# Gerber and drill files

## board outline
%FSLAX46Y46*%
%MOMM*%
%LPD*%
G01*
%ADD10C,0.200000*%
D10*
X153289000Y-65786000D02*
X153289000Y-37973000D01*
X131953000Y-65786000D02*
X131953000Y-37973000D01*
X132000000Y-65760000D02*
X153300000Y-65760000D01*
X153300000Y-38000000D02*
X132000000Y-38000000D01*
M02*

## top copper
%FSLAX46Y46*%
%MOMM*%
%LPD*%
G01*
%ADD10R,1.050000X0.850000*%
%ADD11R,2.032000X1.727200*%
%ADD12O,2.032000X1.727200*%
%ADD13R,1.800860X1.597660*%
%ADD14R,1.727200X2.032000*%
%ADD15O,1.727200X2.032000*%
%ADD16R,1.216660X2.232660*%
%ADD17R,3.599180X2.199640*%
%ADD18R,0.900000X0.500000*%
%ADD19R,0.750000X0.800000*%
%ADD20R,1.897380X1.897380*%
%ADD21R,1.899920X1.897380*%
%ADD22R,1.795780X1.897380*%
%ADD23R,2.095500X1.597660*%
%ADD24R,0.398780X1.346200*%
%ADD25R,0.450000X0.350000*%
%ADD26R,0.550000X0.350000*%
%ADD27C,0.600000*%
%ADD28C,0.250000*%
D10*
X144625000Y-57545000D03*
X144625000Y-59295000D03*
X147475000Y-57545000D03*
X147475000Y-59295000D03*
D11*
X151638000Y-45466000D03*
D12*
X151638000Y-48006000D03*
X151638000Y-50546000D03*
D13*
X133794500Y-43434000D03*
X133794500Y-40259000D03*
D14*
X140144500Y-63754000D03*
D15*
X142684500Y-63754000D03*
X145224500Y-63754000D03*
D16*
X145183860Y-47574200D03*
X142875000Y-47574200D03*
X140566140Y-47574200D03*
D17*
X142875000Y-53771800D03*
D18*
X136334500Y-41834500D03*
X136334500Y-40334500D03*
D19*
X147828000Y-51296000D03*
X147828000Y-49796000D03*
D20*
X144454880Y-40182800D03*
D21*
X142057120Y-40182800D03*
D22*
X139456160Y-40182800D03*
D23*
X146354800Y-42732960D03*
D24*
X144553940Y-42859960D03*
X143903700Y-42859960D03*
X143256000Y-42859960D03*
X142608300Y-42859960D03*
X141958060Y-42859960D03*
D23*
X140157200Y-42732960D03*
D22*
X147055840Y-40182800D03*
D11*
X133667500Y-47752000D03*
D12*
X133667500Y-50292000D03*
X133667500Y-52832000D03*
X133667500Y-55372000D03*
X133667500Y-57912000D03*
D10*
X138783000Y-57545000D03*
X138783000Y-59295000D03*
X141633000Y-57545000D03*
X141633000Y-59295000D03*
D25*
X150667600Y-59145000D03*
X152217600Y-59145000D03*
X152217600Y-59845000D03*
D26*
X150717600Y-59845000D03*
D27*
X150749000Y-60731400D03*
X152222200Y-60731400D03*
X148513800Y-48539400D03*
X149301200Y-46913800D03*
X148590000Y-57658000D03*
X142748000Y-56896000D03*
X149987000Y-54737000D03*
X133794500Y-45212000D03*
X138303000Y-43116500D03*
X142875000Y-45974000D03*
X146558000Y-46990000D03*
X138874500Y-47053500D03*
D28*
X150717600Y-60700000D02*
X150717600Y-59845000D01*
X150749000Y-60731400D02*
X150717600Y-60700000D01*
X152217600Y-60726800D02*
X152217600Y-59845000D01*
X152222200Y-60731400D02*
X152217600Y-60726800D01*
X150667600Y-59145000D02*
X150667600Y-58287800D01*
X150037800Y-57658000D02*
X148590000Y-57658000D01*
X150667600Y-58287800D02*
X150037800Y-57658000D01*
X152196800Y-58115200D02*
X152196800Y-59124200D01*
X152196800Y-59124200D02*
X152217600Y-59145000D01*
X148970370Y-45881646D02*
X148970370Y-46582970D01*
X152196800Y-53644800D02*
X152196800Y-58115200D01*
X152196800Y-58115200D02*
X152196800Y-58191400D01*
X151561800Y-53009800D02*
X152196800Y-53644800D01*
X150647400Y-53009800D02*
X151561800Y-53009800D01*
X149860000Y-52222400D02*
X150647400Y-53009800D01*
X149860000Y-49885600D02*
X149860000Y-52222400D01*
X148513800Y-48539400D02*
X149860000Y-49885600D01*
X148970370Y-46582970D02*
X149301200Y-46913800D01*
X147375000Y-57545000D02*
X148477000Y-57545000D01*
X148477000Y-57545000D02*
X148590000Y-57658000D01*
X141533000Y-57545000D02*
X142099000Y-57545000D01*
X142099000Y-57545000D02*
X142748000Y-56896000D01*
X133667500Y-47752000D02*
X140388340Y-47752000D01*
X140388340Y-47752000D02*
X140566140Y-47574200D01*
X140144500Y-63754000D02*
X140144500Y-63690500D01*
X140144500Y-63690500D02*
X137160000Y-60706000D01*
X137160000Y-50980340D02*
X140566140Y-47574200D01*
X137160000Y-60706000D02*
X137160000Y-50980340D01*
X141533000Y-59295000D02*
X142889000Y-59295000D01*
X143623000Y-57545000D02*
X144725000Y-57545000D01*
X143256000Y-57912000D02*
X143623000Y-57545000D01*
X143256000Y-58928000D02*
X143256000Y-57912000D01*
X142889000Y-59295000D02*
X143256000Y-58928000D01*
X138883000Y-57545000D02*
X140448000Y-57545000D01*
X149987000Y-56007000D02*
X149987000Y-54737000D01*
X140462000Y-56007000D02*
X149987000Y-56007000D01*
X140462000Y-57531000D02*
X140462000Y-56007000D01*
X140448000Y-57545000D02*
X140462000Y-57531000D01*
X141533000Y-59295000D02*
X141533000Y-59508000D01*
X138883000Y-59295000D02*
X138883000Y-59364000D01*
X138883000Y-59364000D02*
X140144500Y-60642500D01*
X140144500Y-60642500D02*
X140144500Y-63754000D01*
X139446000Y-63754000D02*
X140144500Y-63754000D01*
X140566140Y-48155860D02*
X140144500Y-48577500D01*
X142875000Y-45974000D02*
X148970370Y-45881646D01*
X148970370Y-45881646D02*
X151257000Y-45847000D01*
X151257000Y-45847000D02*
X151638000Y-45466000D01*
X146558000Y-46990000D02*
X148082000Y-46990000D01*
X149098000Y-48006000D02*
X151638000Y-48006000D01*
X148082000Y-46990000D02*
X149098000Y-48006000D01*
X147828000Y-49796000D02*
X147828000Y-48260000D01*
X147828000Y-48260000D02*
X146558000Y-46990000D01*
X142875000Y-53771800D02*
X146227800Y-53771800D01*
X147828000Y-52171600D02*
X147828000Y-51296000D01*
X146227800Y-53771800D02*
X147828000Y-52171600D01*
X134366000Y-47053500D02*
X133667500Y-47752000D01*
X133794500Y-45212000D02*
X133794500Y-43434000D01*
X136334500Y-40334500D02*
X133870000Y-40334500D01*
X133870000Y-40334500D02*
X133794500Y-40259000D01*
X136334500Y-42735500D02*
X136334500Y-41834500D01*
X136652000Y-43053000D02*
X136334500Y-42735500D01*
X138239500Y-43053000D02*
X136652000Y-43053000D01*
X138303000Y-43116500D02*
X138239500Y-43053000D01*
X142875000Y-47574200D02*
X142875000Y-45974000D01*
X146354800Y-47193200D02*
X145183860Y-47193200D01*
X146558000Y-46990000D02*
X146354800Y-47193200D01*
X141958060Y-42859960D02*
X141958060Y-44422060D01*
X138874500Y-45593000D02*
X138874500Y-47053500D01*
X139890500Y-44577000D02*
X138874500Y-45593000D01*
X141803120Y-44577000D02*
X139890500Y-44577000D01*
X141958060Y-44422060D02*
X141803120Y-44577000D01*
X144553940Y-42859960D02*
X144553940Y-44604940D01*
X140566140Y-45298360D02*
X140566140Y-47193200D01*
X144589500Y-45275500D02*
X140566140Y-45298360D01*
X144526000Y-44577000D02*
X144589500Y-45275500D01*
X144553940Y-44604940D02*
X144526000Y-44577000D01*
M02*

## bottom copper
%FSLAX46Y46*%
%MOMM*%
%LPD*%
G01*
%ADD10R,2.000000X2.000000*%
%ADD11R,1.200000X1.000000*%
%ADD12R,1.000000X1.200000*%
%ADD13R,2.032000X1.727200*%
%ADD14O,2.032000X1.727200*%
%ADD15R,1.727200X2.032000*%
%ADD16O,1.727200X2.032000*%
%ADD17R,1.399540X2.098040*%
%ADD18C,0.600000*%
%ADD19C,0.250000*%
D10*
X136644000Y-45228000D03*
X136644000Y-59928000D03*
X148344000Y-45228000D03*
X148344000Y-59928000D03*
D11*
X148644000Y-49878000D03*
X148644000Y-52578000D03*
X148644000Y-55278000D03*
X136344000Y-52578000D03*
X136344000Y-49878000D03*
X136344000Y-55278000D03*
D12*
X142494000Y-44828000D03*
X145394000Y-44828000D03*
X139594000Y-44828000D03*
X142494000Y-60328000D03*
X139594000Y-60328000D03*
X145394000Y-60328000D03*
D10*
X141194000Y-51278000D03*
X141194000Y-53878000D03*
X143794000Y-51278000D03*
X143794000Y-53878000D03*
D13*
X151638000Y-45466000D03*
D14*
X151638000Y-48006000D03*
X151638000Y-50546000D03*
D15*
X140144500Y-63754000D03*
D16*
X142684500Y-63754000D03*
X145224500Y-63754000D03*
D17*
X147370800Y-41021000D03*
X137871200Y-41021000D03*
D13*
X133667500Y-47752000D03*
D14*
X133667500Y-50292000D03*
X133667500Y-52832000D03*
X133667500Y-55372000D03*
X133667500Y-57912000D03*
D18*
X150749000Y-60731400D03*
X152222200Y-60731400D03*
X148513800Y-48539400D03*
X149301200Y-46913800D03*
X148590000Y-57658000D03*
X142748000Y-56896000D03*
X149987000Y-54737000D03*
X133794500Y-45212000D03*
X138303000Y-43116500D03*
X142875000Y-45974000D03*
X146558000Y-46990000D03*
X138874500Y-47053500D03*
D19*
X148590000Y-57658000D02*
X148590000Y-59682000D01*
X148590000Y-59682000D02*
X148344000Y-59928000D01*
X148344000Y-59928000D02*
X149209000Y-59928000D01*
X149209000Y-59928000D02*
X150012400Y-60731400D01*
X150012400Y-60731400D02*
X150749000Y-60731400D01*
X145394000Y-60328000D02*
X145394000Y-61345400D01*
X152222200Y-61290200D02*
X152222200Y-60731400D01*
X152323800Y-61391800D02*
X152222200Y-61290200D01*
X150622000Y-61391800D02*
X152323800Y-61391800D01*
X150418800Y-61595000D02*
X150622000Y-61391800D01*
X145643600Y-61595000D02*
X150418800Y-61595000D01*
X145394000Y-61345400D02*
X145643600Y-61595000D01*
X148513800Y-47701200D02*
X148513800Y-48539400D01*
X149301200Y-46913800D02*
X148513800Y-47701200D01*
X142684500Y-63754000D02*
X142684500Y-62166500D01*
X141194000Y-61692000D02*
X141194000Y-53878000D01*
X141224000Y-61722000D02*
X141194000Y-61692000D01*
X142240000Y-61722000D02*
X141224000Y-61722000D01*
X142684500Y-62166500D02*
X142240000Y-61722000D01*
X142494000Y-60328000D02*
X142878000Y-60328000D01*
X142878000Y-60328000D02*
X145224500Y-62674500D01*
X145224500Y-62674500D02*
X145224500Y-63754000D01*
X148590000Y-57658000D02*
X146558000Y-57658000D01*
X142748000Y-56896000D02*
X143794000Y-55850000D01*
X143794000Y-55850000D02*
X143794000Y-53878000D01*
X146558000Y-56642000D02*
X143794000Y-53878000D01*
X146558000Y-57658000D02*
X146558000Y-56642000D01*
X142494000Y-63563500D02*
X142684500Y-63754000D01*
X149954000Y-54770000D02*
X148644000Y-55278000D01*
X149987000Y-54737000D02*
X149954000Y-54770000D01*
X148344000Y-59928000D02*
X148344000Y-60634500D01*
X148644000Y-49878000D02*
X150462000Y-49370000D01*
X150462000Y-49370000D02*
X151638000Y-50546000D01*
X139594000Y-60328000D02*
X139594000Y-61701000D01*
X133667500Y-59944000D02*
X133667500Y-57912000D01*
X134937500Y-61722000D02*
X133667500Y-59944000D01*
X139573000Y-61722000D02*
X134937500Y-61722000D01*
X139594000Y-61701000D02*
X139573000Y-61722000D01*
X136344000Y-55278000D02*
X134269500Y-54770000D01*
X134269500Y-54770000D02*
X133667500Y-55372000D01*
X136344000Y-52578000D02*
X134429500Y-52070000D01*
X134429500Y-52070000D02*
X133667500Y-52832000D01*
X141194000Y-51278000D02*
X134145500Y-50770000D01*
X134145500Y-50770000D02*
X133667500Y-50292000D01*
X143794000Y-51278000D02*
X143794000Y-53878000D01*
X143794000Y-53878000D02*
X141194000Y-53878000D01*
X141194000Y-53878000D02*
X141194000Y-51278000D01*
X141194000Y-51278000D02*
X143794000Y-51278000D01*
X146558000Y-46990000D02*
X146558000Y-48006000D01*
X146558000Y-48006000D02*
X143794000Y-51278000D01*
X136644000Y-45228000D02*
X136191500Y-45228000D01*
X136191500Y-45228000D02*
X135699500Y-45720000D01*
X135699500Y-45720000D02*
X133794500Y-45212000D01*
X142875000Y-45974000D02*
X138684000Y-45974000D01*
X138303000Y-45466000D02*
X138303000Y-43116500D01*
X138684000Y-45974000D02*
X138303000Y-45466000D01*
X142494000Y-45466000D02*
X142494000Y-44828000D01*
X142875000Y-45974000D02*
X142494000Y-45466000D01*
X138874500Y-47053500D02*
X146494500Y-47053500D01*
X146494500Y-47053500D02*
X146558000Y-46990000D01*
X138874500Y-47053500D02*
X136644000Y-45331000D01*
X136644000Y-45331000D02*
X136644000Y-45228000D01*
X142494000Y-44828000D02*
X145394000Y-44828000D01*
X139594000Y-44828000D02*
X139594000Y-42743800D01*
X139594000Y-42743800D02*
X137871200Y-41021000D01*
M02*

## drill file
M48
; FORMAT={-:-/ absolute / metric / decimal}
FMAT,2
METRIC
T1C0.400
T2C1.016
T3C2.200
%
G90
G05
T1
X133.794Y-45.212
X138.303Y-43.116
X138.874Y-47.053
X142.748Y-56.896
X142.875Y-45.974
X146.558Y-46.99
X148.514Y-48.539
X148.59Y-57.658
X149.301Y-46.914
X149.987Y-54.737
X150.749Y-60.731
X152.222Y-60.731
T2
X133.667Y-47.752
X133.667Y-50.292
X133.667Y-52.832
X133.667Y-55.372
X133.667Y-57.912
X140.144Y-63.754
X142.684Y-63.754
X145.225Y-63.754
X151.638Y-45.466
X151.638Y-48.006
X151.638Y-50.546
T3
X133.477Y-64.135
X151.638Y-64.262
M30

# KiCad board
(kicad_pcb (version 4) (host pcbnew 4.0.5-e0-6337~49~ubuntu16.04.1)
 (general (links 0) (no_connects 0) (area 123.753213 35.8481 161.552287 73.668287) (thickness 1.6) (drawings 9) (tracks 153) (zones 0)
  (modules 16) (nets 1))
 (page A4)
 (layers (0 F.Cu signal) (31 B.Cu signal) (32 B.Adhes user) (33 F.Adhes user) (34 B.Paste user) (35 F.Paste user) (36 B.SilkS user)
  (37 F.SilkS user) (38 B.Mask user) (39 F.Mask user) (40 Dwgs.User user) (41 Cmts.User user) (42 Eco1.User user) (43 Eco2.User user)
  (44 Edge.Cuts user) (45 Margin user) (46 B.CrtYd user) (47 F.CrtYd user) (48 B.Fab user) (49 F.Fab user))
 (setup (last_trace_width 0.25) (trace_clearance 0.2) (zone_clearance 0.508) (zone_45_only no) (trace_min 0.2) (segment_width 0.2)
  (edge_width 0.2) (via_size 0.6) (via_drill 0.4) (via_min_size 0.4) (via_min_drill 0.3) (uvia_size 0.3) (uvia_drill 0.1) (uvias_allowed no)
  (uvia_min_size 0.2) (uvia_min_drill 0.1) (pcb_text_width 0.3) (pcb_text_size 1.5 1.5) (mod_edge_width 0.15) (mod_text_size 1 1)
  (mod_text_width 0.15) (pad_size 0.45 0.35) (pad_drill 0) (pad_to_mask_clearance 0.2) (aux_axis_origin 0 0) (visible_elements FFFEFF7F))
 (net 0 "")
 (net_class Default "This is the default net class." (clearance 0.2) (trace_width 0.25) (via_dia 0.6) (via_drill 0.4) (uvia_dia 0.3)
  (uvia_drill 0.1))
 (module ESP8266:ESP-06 (layer B.Cu) (at 142.494 52.578 270)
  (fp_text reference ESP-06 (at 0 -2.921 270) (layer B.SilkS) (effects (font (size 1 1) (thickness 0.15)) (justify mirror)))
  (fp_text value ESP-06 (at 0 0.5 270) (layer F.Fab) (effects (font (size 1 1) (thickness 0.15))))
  (pad GND smd rect (at -7.35 5.85 270) (size 2 2) (layers B.Cu B.Paste B.Mask))
  (pad GP5 smd rect (at 7.35 5.85 270) (size 2 2) (layers B.Cu B.Paste B.Mask))
  (pad GP16 smd rect (at -7.35 -5.85 270) (size 2 2) (layers B.Cu B.Paste B.Mask))
  (pad GP15 smd rect (at 7.35 -5.85 270) (size 2 2) (layers B.Cu B.Paste B.Mask))
  (pad GP14 smd rect (at -2.7 -6.15 270) (size 1 1.2) (layers B.Cu B.Paste B.Mask))
  (pad GP12 smd rect (at 0 -6.15 270) (size 1 1.2) (layers B.Cu B.Paste B.Mask))
  (pad GP13 smd rect (at 2.7 -6.15 270) (size 1 1.2) (layers B.Cu B.Paste B.Mask))
  (pad TX smd rect (at 0 6.15 270) (size 1 1.2) (layers B.Cu B.Paste B.Mask))
  (pad RST smd rect (at -2.7 6.15 270) (size 1 1.2) (layers B.Cu B.Paste B.Mask))
  (pad RX smd rect (at 2.7 6.15 270) (size 1 1.2) (layers B.Cu B.Paste B.Mask))
  (pad 3.3 smd rect (at -7.75 0 270) (size 1.2 1) (layers B.Cu B.Paste B.Mask))
  (pad CHPD smd rect (at -7.75 -2.9 270) (size 1.2 1) (layers B.Cu B.Paste B.Mask))
  (pad ANT smd rect (at -7.75 2.9 270) (size 1.2 1) (layers B.Cu B.Paste B.Mask))
  (pad GP2 smd rect (at 7.75 0 270) (size 1.2 1) (layers B.Cu B.Paste B.Mask))
  (pad GP0 smd rect (at 7.75 2.9 270) (size 1.2 1) (layers B.Cu B.Paste B.Mask))
  (pad GP4 smd rect (at 7.75 -2.9 270) (size 1.2 1) (layers B.Cu B.Paste B.Mask))
  (pad GND smd rect (at -1.3 1.3 270) (size 2 2) (layers B.Cu B.Paste B.Mask))
  (pad GND smd rect (at 1.3 1.3 270) (size 2 2) (layers B.Cu B.Paste B.Mask))
  (pad GND smd rect (at -1.3 -1.3 270) (size 2 2) (layers B.Cu B.Paste B.Mask))
  (pad GND smd rect (at 1.3 -1.3 270) (size 2 2) (layers B.Cu B.Paste B.Mask)))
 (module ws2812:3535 (layer F.Cu) (at 146.05 58.42 180)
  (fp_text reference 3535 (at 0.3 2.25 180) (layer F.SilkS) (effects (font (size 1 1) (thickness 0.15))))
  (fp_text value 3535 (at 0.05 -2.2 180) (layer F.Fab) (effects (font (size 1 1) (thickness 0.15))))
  (pad IN smd rect (at 1.325 0.875 180) (size 1.05 0.85) (drill (offset 0.1 0)) (layers F.Cu F.Paste F.Mask))
  (pad VDD smd rect (at 1.325 -0.875 180) (size 1.05 0.85) (drill (offset 0.1 0)) (layers F.Cu F.Paste F.Mask))
  (pad VSS smd rect (at -1.325 0.875 180) (size 1.05 0.85) (drill (offset -0.1 0)) (layers F.Cu F.Paste F.Mask))
  (pad OUT smd rect (at -1.325 -0.875 180) (size 1.05 0.85) (drill (offset -0.1 0)) (layers F.Cu F.Paste F.Mask)))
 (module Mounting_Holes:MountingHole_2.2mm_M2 (layer F.Cu) (at 133.477 64.135)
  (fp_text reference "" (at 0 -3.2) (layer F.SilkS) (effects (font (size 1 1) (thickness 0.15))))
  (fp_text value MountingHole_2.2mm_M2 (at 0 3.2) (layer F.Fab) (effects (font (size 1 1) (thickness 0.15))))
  (pad 1 np_thru_hole circle (at 0 0) (size 2.2 2.2) (drill 2.2) (layers *.Cu *.Mask F.SilkS)))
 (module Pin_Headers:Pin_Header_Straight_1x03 (layer F.Cu) (at 151.638 45.466)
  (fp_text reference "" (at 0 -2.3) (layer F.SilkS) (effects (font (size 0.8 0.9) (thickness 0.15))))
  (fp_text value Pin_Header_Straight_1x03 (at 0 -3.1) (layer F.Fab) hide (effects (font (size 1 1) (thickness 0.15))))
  (pad 1 thru_hole rect (at 0 0) (size 2.032 1.7272) (drill 1.016) (layers *.Cu *.Mask F.SilkS))
  (pad 2 thru_hole oval (at 0 2.54) (size 2.032 1.7272) (drill 1.016) (layers *.Cu *.Mask F.SilkS))
  (pad 3 thru_hole oval (at 0 5.08) (size 2.032 1.7272) (drill 1.016) (layers *.Cu *.Mask F.SilkS)))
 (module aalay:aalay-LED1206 (layer F.Cu) (at 133.7945 41.8465 90)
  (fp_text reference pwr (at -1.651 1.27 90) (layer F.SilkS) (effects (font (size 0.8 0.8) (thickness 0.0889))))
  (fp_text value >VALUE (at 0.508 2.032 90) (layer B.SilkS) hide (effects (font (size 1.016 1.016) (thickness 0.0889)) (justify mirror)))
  (pad A smd rect (at -1.5875 0 90) (size 1.59766 1.80086) (layers F.Cu F.Paste F.Mask))
  (pad K smd rect (at 1.5875 0 90) (size 1.59766 1.80086) (layers F.Cu F.Paste F.Mask)))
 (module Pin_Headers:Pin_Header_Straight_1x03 (layer F.Cu) (at 140.1445 63.754 90)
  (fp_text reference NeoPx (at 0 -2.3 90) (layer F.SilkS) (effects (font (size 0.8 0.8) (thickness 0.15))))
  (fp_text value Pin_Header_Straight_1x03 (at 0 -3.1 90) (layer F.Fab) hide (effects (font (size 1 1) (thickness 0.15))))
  (pad 1 thru_hole rect (at 0 0 90) (size 2.032 1.7272) (drill 1.016) (layers *.Cu *.Mask F.SilkS))
  (pad 2 thru_hole oval (at 0 2.54 90) (size 2.032 1.7272) (drill 1.016) (layers *.Cu *.Mask F.SilkS))
  (pad 3 thru_hole oval (at 0 5.08 90) (size 2.032 1.7272) (drill 1.016) (layers *.Cu *.Mask F.SilkS)))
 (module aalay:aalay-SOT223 (layer F.Cu) (at 142.875 50.673 180)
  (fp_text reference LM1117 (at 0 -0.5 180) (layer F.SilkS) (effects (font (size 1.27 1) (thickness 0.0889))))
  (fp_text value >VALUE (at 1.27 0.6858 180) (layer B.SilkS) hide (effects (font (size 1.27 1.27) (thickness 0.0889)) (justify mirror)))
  (pad GND smd rect (at -2.30886 3.0988 180) (size 1.21666 2.23266) (layers F.Cu F.Paste F.Mask))
  (pad OUT smd rect (at 0 3.0988 180) (size 1.21666 2.23266) (layers F.Cu F.Paste F.Mask))
  (pad IN smd rect (at 2.30886 3.0988 180) (size 1.21666 2.23266) (layers F.Cu F.Paste F.Mask))
  (pad OUT smd rect (at 0 -3.0988 180) (size 3.59918 2.19964) (layers F.Cu F.Paste F.Mask)))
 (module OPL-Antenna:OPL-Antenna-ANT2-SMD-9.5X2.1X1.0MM (layer B.Cu) (at 142.621 41.021 180)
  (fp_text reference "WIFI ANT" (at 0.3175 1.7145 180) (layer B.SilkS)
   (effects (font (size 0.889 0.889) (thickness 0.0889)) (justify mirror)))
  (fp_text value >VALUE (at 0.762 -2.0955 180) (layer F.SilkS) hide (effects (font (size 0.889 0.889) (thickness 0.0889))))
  (pad 1 smd rect (at -4.7498 0 180) (size 1.39954 2.09804) (layers B.Cu B.Paste B.Mask))
  (pad 2 smd rect (at 4.7498 0 180) (size 1.39954 2.09804) (layers B.Cu B.Paste B.Mask)))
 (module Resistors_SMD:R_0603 (layer F.Cu) (at 136.3345 41.0845 90)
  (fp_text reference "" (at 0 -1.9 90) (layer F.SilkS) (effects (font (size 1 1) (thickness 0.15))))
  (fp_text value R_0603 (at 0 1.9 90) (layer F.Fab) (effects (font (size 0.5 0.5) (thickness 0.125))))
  (pad 1 smd rect (at -0.75 0 90) (size 0.5 0.9) (layers F.Cu F.Paste F.Mask))
  (pad 2 smd rect (at 0.75 0 90) (size 0.5 0.9) (layers F.Cu F.Paste F.Mask)))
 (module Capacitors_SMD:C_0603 (layer F.Cu) (at 147.828 50.546 90)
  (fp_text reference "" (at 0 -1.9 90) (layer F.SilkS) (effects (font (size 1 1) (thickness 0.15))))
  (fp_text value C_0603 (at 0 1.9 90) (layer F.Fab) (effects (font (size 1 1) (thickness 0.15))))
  (pad 1 smd rect (at -0.75 0 90) (size 0.8 0.75) (layers F.Cu F.Paste F.Mask))
  (pad 2 smd rect (at 0.75 0 90) (size 0.8 0.75) (layers F.Cu F.Paste F.Mask)))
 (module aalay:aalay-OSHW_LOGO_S (layer F.Cu) (at 150.622 39.878)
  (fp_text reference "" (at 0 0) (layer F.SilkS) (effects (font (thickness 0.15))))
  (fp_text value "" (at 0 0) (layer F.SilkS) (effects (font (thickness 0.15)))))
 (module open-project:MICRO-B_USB (layer F.Cu) (at 143.256 38.735 180)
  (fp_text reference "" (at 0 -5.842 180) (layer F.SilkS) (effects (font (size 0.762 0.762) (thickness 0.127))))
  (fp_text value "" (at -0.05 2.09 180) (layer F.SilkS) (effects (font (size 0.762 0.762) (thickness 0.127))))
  (pad "" smd rect (at -1.19888 -1.4478 180) (size 1.89738 1.89738) (layers F.Cu F.Paste F.Mask))
  (pad "" smd rect (at 1.19888 -1.4478 180) (size 1.89992 1.89738) (layers F.Cu F.Paste F.Mask))
  (pad "" smd rect (at 3.79984 -1.4478 180) (size 1.79578 1.89738) (layers F.Cu F.Paste F.Mask))
  (pad "" smd rect (at -3.0988 -3.99796 180) (size 2.0955 1.59766) (layers F.Cu F.Paste F.Mask))
  (pad +5 smd rect (at -1.29794 -4.12496 180) (size 0.39878 1.3462) (layers F.Cu F.Paste F.Mask) (clearance 0.2032))
  (pad 2 smd rect (at -0.6477 -4.12496 180) (size 0.39878 1.3462) (layers F.Cu F.Paste F.Mask) (clearance 0.2032))
  (pad 3 smd rect (at 0 -4.12496 180) (size 0.39878 1.3462) (layers F.Cu F.Paste F.Mask) (clearance 0.2032))
  (pad 4 smd rect (at 0.6477 -4.12496 180) (size 0.39878 1.3462) (layers F.Cu F.Paste F.Mask) (clearance 0.2032))
  (pad GND smd rect (at 1.29794 -4.12496 180) (size 0.39878 1.3462) (layers F.Cu F.Paste F.Mask) (clearance 0.2032))
  (pad "" smd rect (at 3.0988 -3.99796 180) (size 2.0955 1.59766) (layers F.Cu F.Paste F.Mask))
  (pad "" smd rect (at -3.79984 -1.4478 180) (size 1.79578 1.89738) (layers F.Cu F.Paste F.Mask)))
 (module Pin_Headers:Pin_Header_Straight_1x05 (layer F.Cu) (at 133.6675 47.752)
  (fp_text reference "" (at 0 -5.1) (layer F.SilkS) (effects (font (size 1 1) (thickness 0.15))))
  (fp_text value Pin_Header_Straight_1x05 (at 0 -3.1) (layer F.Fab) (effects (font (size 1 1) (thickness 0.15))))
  (pad 1 thru_hole rect (at 0 0) (size 2.032 1.7272) (drill 1.016) (layers *.Cu *.Mask F.SilkS))
  (pad 2 thru_hole oval (at 0 2.54) (size 2.032 1.7272) (drill 1.016) (layers *.Cu *.Mask F.SilkS))
  (pad 3 thru_hole oval (at 0 5.08) (size 2.032 1.7272) (drill 1.016) (layers *.Cu *.Mask F.SilkS))
  (pad 4 thru_hole oval (at 0 7.62) (size 2.032 1.7272) (drill 1.016) (layers *.Cu *.Mask F.SilkS))
  (pad 5 thru_hole oval (at 0 10.16) (size 2.032 1.7272) (drill 1.016) (layers *.Cu *.Mask F.SilkS)))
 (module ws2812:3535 (layer F.Cu) (at 140.208 58.42 180)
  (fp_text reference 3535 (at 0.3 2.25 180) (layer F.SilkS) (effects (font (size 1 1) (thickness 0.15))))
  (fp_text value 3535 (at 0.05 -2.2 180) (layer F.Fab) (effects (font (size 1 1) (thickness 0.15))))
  (pad IN smd rect (at 1.325 0.875 180) (size 1.05 0.85) (drill (offset 0.1 0)) (layers F.Cu F.Paste F.Mask))
  (pad VDD smd rect (at 1.325 -0.875 180) (size 1.05 0.85) (drill (offset 0.1 0)) (layers F.Cu F.Paste F.Mask))
  (pad VSS smd rect (at -1.325 0.875 180) (size 1.05 0.85) (drill (offset -0.1 0)) (layers F.Cu F.Paste F.Mask))
  (pad OUT smd rect (at -1.325 -0.875 180) (size 1.05 0.85) (drill (offset -0.1 0)) (layers F.Cu F.Paste F.Mask)))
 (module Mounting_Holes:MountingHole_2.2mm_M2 (layer F.Cu) (at 151.638 64.262)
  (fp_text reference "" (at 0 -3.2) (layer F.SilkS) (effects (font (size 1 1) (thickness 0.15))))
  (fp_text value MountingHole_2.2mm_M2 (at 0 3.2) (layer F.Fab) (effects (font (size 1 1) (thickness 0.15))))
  (pad 1 np_thru_hole circle (at 0 0) (size 2.2 2.2) (drill 2.2) (layers *.Cu *.Mask F.SilkS)))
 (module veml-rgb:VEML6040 (layer F.Cu) (at 151.6126 58.42)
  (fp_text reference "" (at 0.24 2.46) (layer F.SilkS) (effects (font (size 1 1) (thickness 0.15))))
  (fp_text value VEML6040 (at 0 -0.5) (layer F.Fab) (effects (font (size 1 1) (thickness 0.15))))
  (pad GND smd rect (at -0.945 0.725) (size 0.45 0.35) (layers F.Cu F.Paste F.Mask))
  (pad +V smd rect (at 0.605 0.725) (size 0.45 0.35) (layers F.Cu F.Paste F.Mask))
  (pad 3 smd rect (at 0.605 1.425) (size 0.45 0.35) (layers F.Cu F.Paste F.Mask))
  (pad 4 smd rect (at -0.895 1.425) (size 0.55 0.35) (layers F.Cu F.Paste F.Mask)))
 (gr_line (start 153.289 65.786) (end 153.289 37.973) (angle 90) (layer Edge.Cuts) (width 0.2))
 (gr_line (start 131.953 65.786) (end 131.953 37.973) (angle 90) (layer Edge.Cuts) (width 0.2))
 (gr_line (start 132 65.76) (end 153.3 65.76) (angle 90) (layer Edge.Cuts) (width 0.2))
 (gr_line (start 153.3 38) (end 132 38) (angle 90) (layer Edge.Cuts) (width 0.2))
 (segment (start 148.59 57.658) (end 148.59 59.682) (width 0.25) (layer B.Cu) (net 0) (status 800000))
 (segment (start 148.59 59.682) (end 148.344 59.928) (width 0.25) (layer B.Cu) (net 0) (status C00000))
 (segment (start 148.344 59.928) (end 149.209 59.928) (width 0.25) (layer B.Cu) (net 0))
 (segment (start 149.209 59.928) (end 150.0124 60.7314) (width 0.25) (layer B.Cu) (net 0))
 (segment (start 150.7176 60.7) (end 150.7176 59.845) (width 0.25) (layer F.Cu) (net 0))
 (segment (start 150.749 60.7314) (end 150.7176 60.7) (width 0.25) (layer F.Cu) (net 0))
 (via (at 150.749 60.7314) (size 0.6) (drill 0.4) (layers F.Cu B.Cu) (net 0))
 (segment (start 150.0124 60.7314) (end 150.749 60.7314) (width 0.25) (layer B.Cu) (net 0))
 (segment (start 145.394 60.328) (end 145.394 61.3454) (width 0.25) (layer B.Cu) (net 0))
 (segment (start 152.2176 60.7268) (end 152.2176 59.845) (width 0.25) (layer F.Cu) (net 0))
 (segment (start 152.2222 60.7314) (end 152.2176 60.7268) (width 0.25) (layer F.Cu) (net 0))
 (via (at 152.2222 60.7314) (size 0.6) (drill 0.4) (layers F.Cu B.Cu) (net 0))
 (segment (start 152.2222 61.2902) (end 152.2222 60.7314) (width 0.25) (layer B.Cu) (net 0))
 (segment (start 152.3238 61.3918) (end 152.2222 61.2902) (width 0.25) (layer B.Cu) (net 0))
 (segment (start 150.622 61.3918) (end 152.3238 61.3918) (width 0.25) (layer B.Cu) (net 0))
 (segment (start 150.4188 61.595) (end 150.622 61.3918) (width 0.25) (layer B.Cu) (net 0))
 (segment (start 145.6436 61.595) (end 150.4188 61.595) (width 0.25) (layer B.Cu) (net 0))
 (segment (start 145.394 61.3454) (end 145.6436 61.595) (width 0.25) (layer B.Cu) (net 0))
 (segment (start 150.6676 59.145) (end 150.6676 58.2878) (width 0.25) (layer F.Cu) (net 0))
 (segment (start 150.0378 57.658) (end 148.59 57.658) (width 0.25) (layer F.Cu) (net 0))
 (segment (start 150.6676 58.2878) (end 150.0378 57.658) (width 0.25) (layer F.Cu) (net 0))
 (segment (start 152.1968 58.1152) (end 152.1968 59.1242) (width 0.25) (layer F.Cu) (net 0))
 (segment (start 152.1968 59.1242) (end 152.2176 59.145) (width 0.25) (layer F.Cu) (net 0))
 (segment (start 148.97037 45.881646) (end 148.97037 46.58297) (width 0.25) (layer F.Cu) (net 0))
 (segment (start 152.1968 53.6448) (end 152.1968 58.1152) (width 0.25) (layer F.Cu) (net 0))
 (segment (start 152.1968 58.1152) (end 152.1968 58.1914) (width 0.25) (layer F.Cu) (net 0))
 (segment (start 151.5618 53.0098) (end 152.1968 53.6448) (width 0.25) (layer F.Cu) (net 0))
 (segment (start 150.6474 53.0098) (end 151.5618 53.0098) (width 0.25) (layer F.Cu) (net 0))
 (segment (start 149.86 52.2224) (end 150.6474 53.0098) (width 0.25) (layer F.Cu) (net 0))
 (segment (start 149.86 49.8856) (end 149.86 52.2224) (width 0.25) (layer F.Cu) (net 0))
 (segment (start 148.5138 48.5394) (end 149.86 49.8856) (width 0.25) (layer F.Cu) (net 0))
 (via (at 148.5138 48.5394) (size 0.6) (drill 0.4) (layers F.Cu B.Cu) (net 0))
 (segment (start 148.5138 47.7012) (end 148.5138 48.5394) (width 0.25) (layer B.Cu) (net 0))
 (segment (start 149.3012 46.9138) (end 148.5138 47.7012) (width 0.25) (layer B.Cu) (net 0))
 (via (at 149.3012 46.9138) (size 0.6) (drill 0.4) (layers F.Cu B.Cu) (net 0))
 (segment (start 148.97037 46.58297) (end 149.3012 46.9138) (width 0.25) (layer F.Cu) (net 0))
 (segment (start 142.6845 63.754) (end 142.6845 62.1665) (width 0.25) (layer B.Cu) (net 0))
 (segment (start 141.194 61.692) (end 141.194 53.878) (width 0.25) (layer B.Cu) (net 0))
 (segment (start 141.224 61.722) (end 141.194 61.692) (width 0.25) (layer B.Cu) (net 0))
 (segment (start 142.24 61.722) (end 141.224 61.722) (width 0.25) (layer B.Cu) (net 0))
 (segment (start 142.6845 62.1665) (end 142.24 61.722) (width 0.25) (layer B.Cu) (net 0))
 (segment (start 142.494 60.328) (end 142.878 60.328) (width 0.25) (layer B.Cu) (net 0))
 (segment (start 142.878 60.328) (end 145.2245 62.6745) (width 0.25) (layer B.Cu) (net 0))
 (segment (start 145.2245 62.6745) (end 145.2245 63.754) (width 0.25) (layer B.Cu) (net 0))
 (segment (start 147.375 57.545) (end 148.477 57.545) (width 0.25) (layer F.Cu) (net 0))
 (segment (start 148.59 57.658) (end 146.558 57.658) (width 0.25) (layer B.Cu) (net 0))
 (via (at 148.59 57.658) (size 0.6) (drill 0.4) (layers F.Cu B.Cu) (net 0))
 (segment (start 148.477 57.545) (end 148.59 57.658) (width 0.25) (layer F.Cu) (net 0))
 (segment (start 141.533 57.545) (end 142.099 57.545) (width 0.25) (layer F.Cu) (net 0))
 (segment (start 142.099 57.545) (end 142.748 56.896) (width 0.25) (layer F.Cu) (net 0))
 (via (at 142.748 56.896) (size 0.6) (drill 0.4) (layers F.Cu B.Cu) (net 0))
 (segment (start 142.748 56.896) (end 143.794 55.85) (width 0.25) (layer B.Cu) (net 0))
 (segment (start 143.794 55.85) (end 143.794 53.878) (width 0.25) (layer B.Cu) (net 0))
 (segment (start 133.6675 47.752) (end 140.38834 47.752) (width 0.25) (layer F.Cu) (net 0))
 (segment (start 140.38834 47.752) (end 140.56614 47.5742) (width 0.25) (layer F.Cu) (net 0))
 (segment (start 140.1445 63.754) (end 140.1445 63.6905) (width 0.25) (layer F.Cu) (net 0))
 (segment (start 140.1445 63.6905) (end 137.16 60.706) (width 0.25) (layer F.Cu) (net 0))
 (segment (start 137.16 50.98034) (end 140.56614 47.5742) (width 0.25) (layer F.Cu) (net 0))
 (segment (start 137.16 60.706) (end 137.16 50.98034) (width 0.25) (layer F.Cu) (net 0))
 (segment (start 141.533 59.295) (end 142.889 59.295) (width 0.25) (layer F.Cu) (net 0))
 (segment (start 143.623 57.545) (end 144.725 57.545) (width 0.25) (layer F.Cu) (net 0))
 (segment (start 143.256 57.912) (end 143.623 57.545) (width 0.25) (layer F.Cu) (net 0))
 (segment (start 143.256 58.928) (end 143.256 57.912) (width 0.25) (layer F.Cu) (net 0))
 (segment (start 142.889 59.295) (end 143.256 58.928) (width 0.25) (layer F.Cu) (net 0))
 (segment (start 146.558 56.642) (end 143.794 53.878) (width 0.25) (layer B.Cu) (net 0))
 (segment (start 146.558 57.658) (end 146.558 56.642) (width 0.25) (layer B.Cu) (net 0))
 (segment (start 142.494 63.5635) (end 142.6845 63.754) (width 0.25) (layer B.Cu) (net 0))
 (segment (start 138.883 57.545) (end 140.448 57.545) (width 0.25) (layer F.Cu) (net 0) (status 10))
 (segment (start 149.954 54.77) (end 148.644 55.278) (width 0.25) (layer B.Cu) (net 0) (status 20))
 (segment (start 149.987 54.737) (end 149.954 54.77) (width 0.25) (layer B.Cu) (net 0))
 (via (at 149.987 54.737) (size 0.6) (drill 0.4) (layers F.Cu B.Cu) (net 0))
 (segment (start 149.987 56.007) (end 149.987 54.737) (width 0.25) (layer F.Cu) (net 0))
 (segment (start 140.462 56.007) (end 149.987 56.007) (width 0.25) (layer F.Cu) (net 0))
 (segment (start 140.462 57.531) (end 140.462 56.007) (width 0.25) (layer F.Cu) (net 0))
 (segment (start 140.448 57.545) (end 140.462 57.531) (width 0.25) (layer F.Cu) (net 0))
 (segment (start 141.533 59.295) (end 141.533 59.508) (width 0.25) (layer F.Cu) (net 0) (status 30))
 (segment (start 138.883 59.295) (end 138.883 59.364) (width 0.25) (layer F.Cu) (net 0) (status 30))
 (segment (start 138.883 59.364) (end 140.1445 60.6425) (width 0.25) (layer F.Cu) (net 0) (status 10))
 (segment (start 140.1445 60.6425) (end 140.1445 63.754) (width 0.25) (layer F.Cu) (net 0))
 (segment (start 139.446 63.754) (end 140.1445 63.754) (width 0.25) (layer F.Cu) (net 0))
 (segment (start 140.56614 48.15586) (end 140.1445 48.5775) (width 0.25) (layer F.Cu) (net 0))
 (segment (start 148.344 59.928) (end 148.344 60.6345) (width 0.25) (layer B.Cu) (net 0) (status 10))
 (segment (start 148.644 49.878) (end 150.462 49.37) (width 0.25) (layer B.Cu) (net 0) (status 10))
 (segment (start 150.462 49.37) (end 151.638 50.546) (width 0.25) (layer B.Cu) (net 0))
 (segment (start 142.875 45.974) (end 148.97037 45.881646) (width 0.25) (layer F.Cu) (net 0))
 (segment (start 148.97037 45.881646) (end 151.257 45.847) (width 0.25) (layer F.Cu) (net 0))
 (segment (start 151.257 45.847) (end 151.638 45.466) (width 0.25) (layer F.Cu) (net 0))
 (segment (start 146.558 46.99) (end 148.082 46.99) (width 0.25) (layer F.Cu) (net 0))
 (segment (start 149.098 48.006) (end 151.638 48.006) (width 0.25) (layer F.Cu) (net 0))
 (segment (start 148.082 46.99) (end 149.098 48.006) (width 0.25) (layer F.Cu) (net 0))
 (segment (start 147.828 49.796) (end 147.828 48.26) (width 0.25) (layer F.Cu) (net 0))
 (segment (start 147.828 48.26) (end 146.558 46.99) (width 0.25) (layer F.Cu) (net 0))
 (segment (start 142.875 53.7718) (end 146.2278 53.7718) (width 0.25) (layer F.Cu) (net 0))
 (segment (start 147.828 52.1716) (end 147.828 51.296) (width 0.25) (layer F.Cu) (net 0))
 (segment (start 146.2278 53.7718) (end 147.828 52.1716) (width 0.25) (layer F.Cu) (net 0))
 (segment (start 139.594 60.328) (end 139.594 61.701) (width 0.25) (layer B.Cu) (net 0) (status 10))
 (segment (start 133.6675 59.944) (end 133.6675 57.912) (width 0.25) (layer B.Cu) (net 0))
 (segment (start 134.9375 61.722) (end 133.6675 59.944) (width 0.25) (layer B.Cu) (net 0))
 (segment (start 139.573 61.722) (end 134.9375 61.722) (width 0.25) (layer B.Cu) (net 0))
 (segment (start 139.594 61.701) (end 139.573 61.722) (width 0.25) (layer B.Cu) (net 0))
 (segment (start 136.344 55.278) (end 134.2695 54.77) (width 0.25) (layer B.Cu) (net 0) (status 10))
 (segment (start 134.2695 54.77) (end 133.6675 55.372) (width 0.25) (layer B.Cu) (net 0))
 (segment (start 136.344 52.578) (end 134.4295 52.07) (width 0.25) (layer B.Cu) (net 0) (status 10))
 (segment (start 134.4295 52.07) (end 133.6675 52.832) (width 0.25) (layer B.Cu) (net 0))
 (segment (start 141.194 51.278) (end 134.1455 50.77) (width 0.25) (layer B.Cu) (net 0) (status 10))
 (segment (start 134.1455 50.77) (end 133.6675 50.292) (width 0.25) (layer B.Cu) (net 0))
 (segment (start 134.366 47.0535) (end 133.6675 47.752) (width 0.25) (layer F.Cu) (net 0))
 (segment (start 143.794 51.278) (end 143.794 53.878) (width 0.25) (layer B.Cu) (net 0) (status 30))
 (segment (start 143.794 53.878) (end 141.194 53.878) (width 0.25) (layer B.Cu) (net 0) (status 30))
 (segment (start 141.194 53.878) (end 141.194 51.278) (width 0.25) (layer B.Cu) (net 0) (status 30))
 (segment (start 141.194 51.278) (end 143.794 51.278) (width 0.25) (layer B.Cu) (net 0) (status 30))
 (segment (start 146.558 46.99) (end 146.558 48.006) (width 0.25) (layer B.Cu) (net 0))
 (segment (start 146.558 48.006) (end 143.794 51.278) (width 0.25) (layer B.Cu) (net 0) (status 20))
 (segment (start 136.644 45.228) (end 136.1915 45.228) (width 0.25) (layer B.Cu) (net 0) (status 30))
 (segment (start 136.1915 45.228) (end 135.6995 45.72) (width 0.25) (layer B.Cu) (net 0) (status 30))
 (segment (start 135.6995 45.72) (end 133.7945 45.212) (width 0.25) (layer B.Cu) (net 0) (status 10))
 (via (at 133.7945 45.212) (size 0.6) (drill 0.4) (layers F.Cu B.Cu) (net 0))
 (segment (start 133.7945 45.212) (end 133.7945 43.434) (width 0.25) (layer F.Cu) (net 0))
 (segment (start 136.3345 40.3345) (end 133.87 40.3345) (width 0.25) (layer F.Cu) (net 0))
 (segment (start 133.87 40.3345) (end 133.7945 40.259) (width 0.25) (layer F.Cu) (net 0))
 (segment (start 142.875 45.974) (end 138.684 45.974) (width 0.25) (layer B.Cu) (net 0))
 (segment (start 136.3345 42.7355) (end 136.3345 41.8345) (width 0.25) (layer F.Cu) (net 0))
 (segment (start 136.652 43.053) (end 136.3345 42.7355) (width 0.25) (layer F.Cu) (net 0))
 (segment (start 138.2395 43.053) (end 136.652 43.053) (width 0.25) (layer F.Cu) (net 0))
 (segment (start 138.303 43.1165) (end 138.2395 43.053) (width 0.25) (layer F.Cu) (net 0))
 (via (at 138.303 43.1165) (size 0.6) (drill 0.4) (layers F.Cu B.Cu) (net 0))
 (segment (start 138.303 45.466) (end 138.303 43.1165) (width 0.25) (layer B.Cu) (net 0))
 (segment (start 138.684 45.974) (end 138.303 45.466) (width 0.25) (layer B.Cu) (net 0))
 (segment (start 142.875 47.5742) (end 142.875 45.974) (width 0.25) (layer F.Cu) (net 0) (status 10))
 (segment (start 142.494 45.466) (end 142.494 44.828) (width 0.25) (layer B.Cu) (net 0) (status 20))
 (segment (start 142.875 45.974) (end 142.494 45.466) (width 0.25) (layer B.Cu) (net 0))
 (via (at 142.875 45.974) (size 0.6) (drill 0.4) (layers F.Cu B.Cu) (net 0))
 (segment (start 138.8745 47.0535) (end 146.4945 47.0535) (width 0.25) (layer B.Cu) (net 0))
 (segment (start 146.3548 47.1932) (end 145.18386 47.1932) (width 0.25) (layer F.Cu) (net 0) (status 20))
 (segment (start 146.558 46.99) (end 146.3548 47.1932) (width 0.25) (layer F.Cu) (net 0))
 (via (at 146.558 46.99) (size 0.6) (drill 0.4) (layers F.Cu B.Cu) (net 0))
 (segment (start 146.4945 47.0535) (end 146.558 46.99) (width 0.25) (layer B.Cu) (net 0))
 (segment (start 141.95806 42.85996) (end 141.95806 44.42206) (width 0.25) (layer F.Cu) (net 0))
 (segment (start 138.8745 47.0535) (end 136.644 45.331) (width 0.25) (layer B.Cu) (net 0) (status 20))
 (via (at 138.8745 47.0535) (size 0.6) (drill 0.4) (layers F.Cu B.Cu) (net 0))
 (segment (start 138.8745 45.593) (end 138.8745 47.0535) (width 0.25) (layer F.Cu) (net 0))
 (segment (start 139.8905 44.577) (end 138.8745 45.593) (width 0.25) (layer F.Cu) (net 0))
 (segment (start 141.80312 44.577) (end 139.8905 44.577) (width 0.25) (layer F.Cu) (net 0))
 (segment (start 141.95806 44.42206) (end 141.80312 44.577) (width 0.25) (layer F.Cu) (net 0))
 (segment (start 136.644 45.331) (end 136.644 45.228) (width 0.25) (layer B.Cu) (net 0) (status 30))
 (segment (start 144.55394 42.85996) (end 144.55394 44.60494) (width 0.25) (layer F.Cu) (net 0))
 (segment (start 140.56614 45.29836) (end 140.56614 47.1932) (width 0.25) (layer F.Cu) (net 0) (status 20))
 (segment (start 144.5895 45.2755) (end 140.56614 45.29836) (width 0.25) (layer F.Cu) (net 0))
 (segment (start 144.526 44.577) (end 144.5895 45.2755) (width 0.25) (layer F.Cu) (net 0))
 (segment (start 144.55394 44.60494) (end 144.526 44.577) (width 0.25) (layer F.Cu) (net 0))
 (segment (start 142.494 44.828) (end 145.394 44.828) (width 0.25) (layer B.Cu) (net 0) (status 30))
 (segment (start 139.594 44.828) (end 139.594 42.7438) (width 0.25) (layer B.Cu) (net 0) (status 10))
 (segment (start 139.594 42.7438) (end 137.8712 41.021) (width 0.25) (layer B.Cu) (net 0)))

